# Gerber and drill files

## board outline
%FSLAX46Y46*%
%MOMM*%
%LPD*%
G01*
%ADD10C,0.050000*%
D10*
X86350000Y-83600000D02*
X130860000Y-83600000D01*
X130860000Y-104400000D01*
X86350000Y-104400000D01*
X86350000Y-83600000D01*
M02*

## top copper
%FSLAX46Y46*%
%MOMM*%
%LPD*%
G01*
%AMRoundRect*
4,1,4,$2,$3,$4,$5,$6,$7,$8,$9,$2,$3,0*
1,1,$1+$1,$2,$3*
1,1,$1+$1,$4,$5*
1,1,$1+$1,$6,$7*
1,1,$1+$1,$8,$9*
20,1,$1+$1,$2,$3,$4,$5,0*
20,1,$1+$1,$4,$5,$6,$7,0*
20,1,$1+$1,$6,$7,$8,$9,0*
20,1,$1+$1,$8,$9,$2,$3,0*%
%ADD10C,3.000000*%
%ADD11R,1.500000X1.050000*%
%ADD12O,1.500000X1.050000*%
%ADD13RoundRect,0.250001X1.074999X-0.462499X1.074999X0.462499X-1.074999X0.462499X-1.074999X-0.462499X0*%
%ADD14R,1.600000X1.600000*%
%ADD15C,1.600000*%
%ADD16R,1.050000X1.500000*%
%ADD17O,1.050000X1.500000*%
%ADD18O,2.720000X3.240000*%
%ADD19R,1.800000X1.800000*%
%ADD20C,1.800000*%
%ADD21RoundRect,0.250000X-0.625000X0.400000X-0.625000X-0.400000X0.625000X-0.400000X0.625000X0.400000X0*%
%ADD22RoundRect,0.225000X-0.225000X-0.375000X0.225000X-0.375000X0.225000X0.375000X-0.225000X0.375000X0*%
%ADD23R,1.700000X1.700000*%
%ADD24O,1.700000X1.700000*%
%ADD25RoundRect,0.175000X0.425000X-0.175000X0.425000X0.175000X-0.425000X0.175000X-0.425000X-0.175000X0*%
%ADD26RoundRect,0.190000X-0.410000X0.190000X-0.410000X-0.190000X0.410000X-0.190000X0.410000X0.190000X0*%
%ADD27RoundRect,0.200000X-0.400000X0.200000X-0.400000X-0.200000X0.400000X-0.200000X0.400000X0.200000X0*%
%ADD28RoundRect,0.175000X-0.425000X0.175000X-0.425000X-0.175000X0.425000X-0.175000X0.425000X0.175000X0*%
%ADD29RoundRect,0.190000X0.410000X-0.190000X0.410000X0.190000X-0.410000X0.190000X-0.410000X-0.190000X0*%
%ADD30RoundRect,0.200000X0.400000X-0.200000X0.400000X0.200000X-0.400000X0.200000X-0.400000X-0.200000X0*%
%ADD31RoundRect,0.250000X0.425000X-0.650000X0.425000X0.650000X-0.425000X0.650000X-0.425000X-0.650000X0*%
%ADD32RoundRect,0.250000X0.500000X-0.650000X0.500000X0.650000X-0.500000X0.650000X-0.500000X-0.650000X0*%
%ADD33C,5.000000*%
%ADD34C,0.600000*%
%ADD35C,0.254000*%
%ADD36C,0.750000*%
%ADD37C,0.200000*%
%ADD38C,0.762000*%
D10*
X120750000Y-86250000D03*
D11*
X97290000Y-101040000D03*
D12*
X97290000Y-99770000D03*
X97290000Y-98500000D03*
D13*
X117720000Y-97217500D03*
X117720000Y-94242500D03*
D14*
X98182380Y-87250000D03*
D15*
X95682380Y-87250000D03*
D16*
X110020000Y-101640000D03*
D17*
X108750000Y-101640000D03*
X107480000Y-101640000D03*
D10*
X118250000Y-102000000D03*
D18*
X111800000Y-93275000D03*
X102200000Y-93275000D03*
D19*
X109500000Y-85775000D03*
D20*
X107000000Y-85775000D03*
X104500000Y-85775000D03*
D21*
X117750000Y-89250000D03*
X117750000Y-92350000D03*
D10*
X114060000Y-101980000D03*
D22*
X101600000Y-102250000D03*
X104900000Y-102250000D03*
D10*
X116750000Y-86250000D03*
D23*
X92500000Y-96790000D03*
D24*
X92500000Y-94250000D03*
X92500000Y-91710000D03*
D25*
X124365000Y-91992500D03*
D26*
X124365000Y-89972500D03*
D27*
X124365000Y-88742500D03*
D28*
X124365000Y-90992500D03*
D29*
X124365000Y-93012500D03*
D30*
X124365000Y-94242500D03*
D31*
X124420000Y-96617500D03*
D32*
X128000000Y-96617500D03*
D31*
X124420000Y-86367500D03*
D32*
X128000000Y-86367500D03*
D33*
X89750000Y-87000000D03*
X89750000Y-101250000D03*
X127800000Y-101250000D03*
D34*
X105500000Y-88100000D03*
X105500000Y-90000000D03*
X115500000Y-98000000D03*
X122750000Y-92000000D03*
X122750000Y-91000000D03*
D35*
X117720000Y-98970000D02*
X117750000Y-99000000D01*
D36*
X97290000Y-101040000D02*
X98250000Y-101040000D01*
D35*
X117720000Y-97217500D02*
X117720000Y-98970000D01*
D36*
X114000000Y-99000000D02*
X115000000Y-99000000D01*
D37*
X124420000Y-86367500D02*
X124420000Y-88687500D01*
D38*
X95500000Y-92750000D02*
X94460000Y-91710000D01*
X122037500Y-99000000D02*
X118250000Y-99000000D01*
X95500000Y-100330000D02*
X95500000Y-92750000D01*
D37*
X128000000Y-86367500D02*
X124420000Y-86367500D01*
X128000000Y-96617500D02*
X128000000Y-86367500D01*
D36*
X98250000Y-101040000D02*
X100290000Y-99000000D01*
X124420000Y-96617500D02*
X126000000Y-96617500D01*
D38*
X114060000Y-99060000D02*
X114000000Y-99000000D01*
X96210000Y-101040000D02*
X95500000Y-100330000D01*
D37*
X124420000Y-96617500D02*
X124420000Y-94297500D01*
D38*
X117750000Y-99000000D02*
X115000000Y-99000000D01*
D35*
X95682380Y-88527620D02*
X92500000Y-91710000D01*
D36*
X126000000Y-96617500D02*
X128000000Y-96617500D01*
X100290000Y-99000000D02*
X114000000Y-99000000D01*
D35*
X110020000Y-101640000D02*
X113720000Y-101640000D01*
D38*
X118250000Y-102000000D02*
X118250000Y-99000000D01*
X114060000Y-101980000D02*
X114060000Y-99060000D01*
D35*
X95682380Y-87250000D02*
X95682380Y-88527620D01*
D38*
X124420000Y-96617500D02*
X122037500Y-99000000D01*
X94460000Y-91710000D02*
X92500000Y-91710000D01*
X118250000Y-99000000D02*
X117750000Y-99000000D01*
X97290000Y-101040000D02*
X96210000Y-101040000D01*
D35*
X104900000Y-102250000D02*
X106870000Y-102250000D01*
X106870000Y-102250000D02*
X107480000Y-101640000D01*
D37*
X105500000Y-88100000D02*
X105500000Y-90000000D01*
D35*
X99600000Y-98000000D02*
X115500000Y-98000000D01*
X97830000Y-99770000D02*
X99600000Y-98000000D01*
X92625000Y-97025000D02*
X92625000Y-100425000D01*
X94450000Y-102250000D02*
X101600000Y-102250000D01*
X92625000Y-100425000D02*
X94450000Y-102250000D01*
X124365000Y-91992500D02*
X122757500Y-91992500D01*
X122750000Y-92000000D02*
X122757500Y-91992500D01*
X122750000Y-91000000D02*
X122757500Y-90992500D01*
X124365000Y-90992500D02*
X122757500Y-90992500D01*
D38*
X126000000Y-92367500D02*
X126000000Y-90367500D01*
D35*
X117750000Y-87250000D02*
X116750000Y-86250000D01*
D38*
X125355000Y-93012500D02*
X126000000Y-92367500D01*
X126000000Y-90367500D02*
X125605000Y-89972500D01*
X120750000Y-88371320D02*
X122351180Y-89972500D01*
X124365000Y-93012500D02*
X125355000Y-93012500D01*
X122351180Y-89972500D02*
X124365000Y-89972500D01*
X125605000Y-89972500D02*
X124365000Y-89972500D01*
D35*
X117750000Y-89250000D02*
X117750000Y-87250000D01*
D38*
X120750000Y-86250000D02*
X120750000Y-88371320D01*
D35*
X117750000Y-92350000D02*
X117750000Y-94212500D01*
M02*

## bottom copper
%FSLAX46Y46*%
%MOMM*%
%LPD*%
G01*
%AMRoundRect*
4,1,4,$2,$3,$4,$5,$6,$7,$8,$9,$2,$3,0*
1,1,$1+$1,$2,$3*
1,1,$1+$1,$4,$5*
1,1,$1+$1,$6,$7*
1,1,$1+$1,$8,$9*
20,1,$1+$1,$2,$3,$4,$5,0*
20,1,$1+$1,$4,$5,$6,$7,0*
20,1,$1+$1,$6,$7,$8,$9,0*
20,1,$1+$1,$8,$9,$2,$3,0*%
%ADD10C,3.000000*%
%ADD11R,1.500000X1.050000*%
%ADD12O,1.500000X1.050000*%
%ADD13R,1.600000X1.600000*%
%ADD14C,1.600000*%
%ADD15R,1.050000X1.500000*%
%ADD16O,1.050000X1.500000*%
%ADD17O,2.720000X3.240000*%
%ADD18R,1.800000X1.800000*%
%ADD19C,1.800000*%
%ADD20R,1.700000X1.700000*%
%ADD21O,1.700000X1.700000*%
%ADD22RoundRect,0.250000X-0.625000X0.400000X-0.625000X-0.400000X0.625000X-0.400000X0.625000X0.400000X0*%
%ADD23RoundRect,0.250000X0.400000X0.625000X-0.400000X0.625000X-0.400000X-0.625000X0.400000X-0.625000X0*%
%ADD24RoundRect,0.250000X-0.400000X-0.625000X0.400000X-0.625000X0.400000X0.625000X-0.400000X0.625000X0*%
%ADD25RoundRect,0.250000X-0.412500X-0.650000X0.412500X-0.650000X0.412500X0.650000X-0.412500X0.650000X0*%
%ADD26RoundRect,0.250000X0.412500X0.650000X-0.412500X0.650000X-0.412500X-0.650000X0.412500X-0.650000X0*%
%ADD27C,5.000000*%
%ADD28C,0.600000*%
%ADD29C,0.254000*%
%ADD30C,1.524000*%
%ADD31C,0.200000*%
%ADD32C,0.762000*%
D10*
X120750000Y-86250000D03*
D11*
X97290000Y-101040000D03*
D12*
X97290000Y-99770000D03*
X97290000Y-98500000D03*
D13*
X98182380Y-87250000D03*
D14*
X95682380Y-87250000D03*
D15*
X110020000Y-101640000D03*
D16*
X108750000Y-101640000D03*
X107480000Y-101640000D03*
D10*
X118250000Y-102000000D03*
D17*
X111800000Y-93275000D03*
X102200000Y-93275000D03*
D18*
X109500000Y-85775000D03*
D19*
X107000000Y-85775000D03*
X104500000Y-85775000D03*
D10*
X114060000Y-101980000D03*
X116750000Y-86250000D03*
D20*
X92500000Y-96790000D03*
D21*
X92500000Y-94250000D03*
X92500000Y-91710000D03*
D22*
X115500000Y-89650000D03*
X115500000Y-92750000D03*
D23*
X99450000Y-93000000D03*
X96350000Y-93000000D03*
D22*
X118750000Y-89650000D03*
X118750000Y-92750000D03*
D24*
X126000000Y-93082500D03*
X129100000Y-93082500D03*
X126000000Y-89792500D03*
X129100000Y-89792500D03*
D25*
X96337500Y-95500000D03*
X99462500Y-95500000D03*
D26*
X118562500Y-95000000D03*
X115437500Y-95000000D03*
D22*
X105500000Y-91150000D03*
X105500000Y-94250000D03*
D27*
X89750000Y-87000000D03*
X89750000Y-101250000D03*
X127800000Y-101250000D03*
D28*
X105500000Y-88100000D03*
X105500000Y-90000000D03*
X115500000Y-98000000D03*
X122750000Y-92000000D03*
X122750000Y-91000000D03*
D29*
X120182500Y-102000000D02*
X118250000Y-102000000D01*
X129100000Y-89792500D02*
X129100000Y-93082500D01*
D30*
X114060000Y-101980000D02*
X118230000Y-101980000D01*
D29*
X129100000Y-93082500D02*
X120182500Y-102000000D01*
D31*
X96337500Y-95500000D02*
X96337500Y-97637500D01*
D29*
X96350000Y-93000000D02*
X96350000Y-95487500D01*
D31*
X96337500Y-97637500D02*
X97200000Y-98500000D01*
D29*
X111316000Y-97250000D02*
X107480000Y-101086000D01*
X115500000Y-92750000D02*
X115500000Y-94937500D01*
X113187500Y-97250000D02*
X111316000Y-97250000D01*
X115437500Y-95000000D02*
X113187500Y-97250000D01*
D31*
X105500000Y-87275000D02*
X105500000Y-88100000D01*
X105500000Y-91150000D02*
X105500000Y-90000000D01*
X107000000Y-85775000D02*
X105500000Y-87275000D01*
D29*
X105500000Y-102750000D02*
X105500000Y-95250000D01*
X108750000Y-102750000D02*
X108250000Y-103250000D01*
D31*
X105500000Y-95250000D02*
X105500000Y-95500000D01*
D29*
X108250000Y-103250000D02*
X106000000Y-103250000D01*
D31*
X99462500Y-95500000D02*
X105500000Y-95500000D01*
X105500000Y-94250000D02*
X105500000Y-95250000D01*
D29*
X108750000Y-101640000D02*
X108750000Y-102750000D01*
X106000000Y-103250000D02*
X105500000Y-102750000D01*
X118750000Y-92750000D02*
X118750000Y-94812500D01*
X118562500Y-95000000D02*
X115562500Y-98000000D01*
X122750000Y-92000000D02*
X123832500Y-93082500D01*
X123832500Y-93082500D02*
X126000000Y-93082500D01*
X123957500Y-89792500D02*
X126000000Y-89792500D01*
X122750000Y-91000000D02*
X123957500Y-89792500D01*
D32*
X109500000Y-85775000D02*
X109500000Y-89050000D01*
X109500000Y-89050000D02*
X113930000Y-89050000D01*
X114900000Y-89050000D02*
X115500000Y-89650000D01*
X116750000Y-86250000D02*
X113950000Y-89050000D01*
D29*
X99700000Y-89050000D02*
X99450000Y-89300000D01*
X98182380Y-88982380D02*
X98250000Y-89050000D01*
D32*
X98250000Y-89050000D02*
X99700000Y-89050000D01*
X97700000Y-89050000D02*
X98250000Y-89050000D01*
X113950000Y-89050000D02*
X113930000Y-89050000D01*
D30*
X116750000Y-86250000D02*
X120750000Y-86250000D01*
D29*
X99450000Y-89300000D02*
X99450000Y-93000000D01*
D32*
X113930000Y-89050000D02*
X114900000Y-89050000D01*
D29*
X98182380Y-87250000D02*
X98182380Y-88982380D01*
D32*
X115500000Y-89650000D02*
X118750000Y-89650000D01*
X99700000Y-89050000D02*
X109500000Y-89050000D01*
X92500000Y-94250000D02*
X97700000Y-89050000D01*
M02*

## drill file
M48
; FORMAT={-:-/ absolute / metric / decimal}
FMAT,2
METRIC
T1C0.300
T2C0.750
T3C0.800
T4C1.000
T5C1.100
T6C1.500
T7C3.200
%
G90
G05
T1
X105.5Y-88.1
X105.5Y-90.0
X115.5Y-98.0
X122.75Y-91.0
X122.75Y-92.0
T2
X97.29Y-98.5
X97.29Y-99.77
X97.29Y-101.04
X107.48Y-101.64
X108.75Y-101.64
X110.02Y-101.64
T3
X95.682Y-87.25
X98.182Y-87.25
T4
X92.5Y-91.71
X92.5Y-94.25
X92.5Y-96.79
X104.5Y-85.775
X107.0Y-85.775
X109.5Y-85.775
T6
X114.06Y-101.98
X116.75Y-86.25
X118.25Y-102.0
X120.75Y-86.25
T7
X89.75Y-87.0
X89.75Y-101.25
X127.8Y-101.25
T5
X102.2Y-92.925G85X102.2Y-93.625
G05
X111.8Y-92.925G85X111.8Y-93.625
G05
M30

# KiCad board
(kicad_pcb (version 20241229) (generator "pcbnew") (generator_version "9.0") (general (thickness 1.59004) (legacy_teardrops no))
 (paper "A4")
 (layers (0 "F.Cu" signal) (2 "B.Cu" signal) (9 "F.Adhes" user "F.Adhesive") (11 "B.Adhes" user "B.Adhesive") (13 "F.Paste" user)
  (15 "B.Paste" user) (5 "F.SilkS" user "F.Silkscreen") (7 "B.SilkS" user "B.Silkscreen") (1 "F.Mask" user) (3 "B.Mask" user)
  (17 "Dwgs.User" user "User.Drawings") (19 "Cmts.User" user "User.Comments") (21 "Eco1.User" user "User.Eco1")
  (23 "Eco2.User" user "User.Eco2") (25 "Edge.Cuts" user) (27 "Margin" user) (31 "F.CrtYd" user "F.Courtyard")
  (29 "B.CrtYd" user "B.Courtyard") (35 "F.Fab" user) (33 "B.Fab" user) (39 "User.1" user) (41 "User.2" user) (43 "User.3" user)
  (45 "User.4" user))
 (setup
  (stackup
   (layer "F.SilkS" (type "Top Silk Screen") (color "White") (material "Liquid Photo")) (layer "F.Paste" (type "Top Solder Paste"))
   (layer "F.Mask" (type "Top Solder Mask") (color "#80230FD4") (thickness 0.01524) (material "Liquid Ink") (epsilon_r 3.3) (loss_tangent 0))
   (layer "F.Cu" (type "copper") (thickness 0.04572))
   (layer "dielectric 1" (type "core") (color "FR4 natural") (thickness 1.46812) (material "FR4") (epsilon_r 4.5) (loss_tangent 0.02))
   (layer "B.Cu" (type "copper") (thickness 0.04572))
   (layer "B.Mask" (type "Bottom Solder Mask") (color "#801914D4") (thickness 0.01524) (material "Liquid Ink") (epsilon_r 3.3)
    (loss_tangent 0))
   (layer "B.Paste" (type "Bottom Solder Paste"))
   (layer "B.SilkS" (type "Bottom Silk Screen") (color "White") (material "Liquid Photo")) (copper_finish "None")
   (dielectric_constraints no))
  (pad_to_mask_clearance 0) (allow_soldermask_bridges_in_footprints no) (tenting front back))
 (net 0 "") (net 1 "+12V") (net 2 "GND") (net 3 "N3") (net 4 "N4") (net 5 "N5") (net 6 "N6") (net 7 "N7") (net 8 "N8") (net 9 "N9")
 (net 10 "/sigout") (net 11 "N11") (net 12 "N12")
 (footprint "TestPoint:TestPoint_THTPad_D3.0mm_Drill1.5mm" (layer "F.Cu") (at 120.75 86.25)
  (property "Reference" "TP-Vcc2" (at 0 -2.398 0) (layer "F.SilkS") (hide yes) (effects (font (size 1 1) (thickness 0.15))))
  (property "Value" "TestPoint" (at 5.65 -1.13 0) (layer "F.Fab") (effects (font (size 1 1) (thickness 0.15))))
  (pad "1" thru_hole circle (at 0 0) (size 3 3) (drill 1.5) (layers "*.Cu" "*.Mask") (remove_unused_layers no) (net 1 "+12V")))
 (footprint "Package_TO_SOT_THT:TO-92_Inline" (layer "F.Cu") (at 97.29 101.04 90)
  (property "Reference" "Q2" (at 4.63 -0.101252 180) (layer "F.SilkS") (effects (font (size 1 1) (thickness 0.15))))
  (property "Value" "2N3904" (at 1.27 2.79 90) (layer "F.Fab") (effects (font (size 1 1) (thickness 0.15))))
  (pad "1" thru_hole rect (at 0 0 90) (size 1.05 1.5) (drill 0.75) (layers "*.Cu" "*.Mask") (remove_unused_layers no) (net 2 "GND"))
  (pad "2" thru_hole oval (at 1.27 0 90) (size 1.05 1.5) (drill 0.75) (layers "*.Cu" "*.Mask") (remove_unused_layers no) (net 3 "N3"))
  (pad "3" thru_hole oval (at 2.54 0 90) (size 1.05 1.5) (drill 0.75) (layers "*.Cu" "*.Mask") (remove_unused_layers no) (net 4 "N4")))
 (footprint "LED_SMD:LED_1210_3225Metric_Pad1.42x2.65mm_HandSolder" (layer "F.Cu") (at 117.72 95.73 90)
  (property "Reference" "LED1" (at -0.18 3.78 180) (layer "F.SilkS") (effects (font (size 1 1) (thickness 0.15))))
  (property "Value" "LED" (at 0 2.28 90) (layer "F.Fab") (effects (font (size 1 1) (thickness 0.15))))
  (pad "1" smd roundrect (at -1.4875 0 90) (size 1.425 2.65) (layers "F.Cu" "F.Mask" "F.Paste") (roundrect_rratio 0.175439) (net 2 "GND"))
  (pad "2" smd roundrect (at 1.4875 0 90) (size 1.425 2.65) (layers "F.Cu" "F.Mask" "F.Paste") (roundrect_rratio 0.175439) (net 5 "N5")))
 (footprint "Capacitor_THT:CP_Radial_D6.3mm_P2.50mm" (layer "F.Cu") (at 98.18238 87.25 180)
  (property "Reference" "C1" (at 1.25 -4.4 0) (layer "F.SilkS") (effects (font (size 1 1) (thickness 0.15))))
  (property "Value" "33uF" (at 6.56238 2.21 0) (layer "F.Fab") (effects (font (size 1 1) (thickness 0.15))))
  (pad "1" thru_hole rect (at 0 0 180) (size 1.6 1.6) (drill 0.8) (layers "*.Cu" "*.Mask") (remove_unused_layers no) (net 1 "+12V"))
  (pad "2" thru_hole circle (at 2.5 0 180) (size 1.6 1.6) (drill 0.8) (layers "*.Cu" "*.Mask") (remove_unused_layers no) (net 2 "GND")))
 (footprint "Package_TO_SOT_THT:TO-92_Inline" (layer "F.Cu") (at 110.02 101.64 180)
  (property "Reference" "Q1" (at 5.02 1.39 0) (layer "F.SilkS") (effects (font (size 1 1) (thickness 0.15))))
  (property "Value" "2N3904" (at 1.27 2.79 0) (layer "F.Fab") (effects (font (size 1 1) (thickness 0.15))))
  (pad "1" thru_hole rect (at 0 0 180) (size 1.05 1.5) (drill 0.75) (layers "*.Cu" "*.Mask") (remove_unused_layers no) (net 2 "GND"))
  (pad "2" thru_hole oval (at 1.27 0 180) (size 1.05 1.5) (drill 0.75) (layers "*.Cu" "*.Mask") (remove_unused_layers no) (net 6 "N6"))
  (pad "3" thru_hole oval (at 2.54 0 180) (size 1.05 1.5) (drill 0.75) (layers "*.Cu" "*.Mask") (remove_unused_layers no) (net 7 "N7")))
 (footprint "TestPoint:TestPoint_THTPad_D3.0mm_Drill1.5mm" (layer "F.Cu") (at 118.25 102)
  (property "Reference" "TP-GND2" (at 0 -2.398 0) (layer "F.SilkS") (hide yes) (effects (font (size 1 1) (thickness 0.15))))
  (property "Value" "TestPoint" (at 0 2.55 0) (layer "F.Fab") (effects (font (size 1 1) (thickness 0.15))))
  (pad "1" thru_hole circle (at 0 0) (size 3 3) (drill 1.5) (layers "*.Cu" "*.Mask") (remove_unused_layers no) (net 2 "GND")))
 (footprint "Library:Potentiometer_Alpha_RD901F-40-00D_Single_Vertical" (layer "F.Cu") (at 109.5 85.775 -90)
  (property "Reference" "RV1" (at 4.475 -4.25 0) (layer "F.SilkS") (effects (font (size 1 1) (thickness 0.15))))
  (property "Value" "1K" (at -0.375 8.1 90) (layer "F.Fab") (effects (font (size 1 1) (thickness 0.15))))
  (pad "" thru_hole oval (at 7.5 -2.3) (size 2.72 3.24) (drill oval 1.1 1.8) (layers "*.Cu" "*.Mask") (remove_unused_layers no))
  (pad "" thru_hole oval (at 7.5 7.3) (size 2.72 3.24) (drill oval 1.1 1.8) (layers "*.Cu" "*.Mask") (remove_unused_layers no))
  (pad "1" thru_hole rect (at 0 0) (size 1.8 1.8) (drill 1) (layers "*.Cu" "*.Mask") (remove_unused_layers no) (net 1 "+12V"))
  (pad "2" thru_hole circle (at 0 2.5) (size 1.8 1.8) (drill 1) (layers "*.Cu" "*.Mask") (remove_unused_layers no) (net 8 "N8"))
  (pad "3" thru_hole circle (at 0 5) (size 1.8 1.8) (drill 1) (layers "*.Cu" "*.Mask") (remove_unused_layers no) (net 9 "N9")))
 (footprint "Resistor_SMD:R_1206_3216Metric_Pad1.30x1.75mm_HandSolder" (layer "F.Cu") (at 117.75 90.8 -90)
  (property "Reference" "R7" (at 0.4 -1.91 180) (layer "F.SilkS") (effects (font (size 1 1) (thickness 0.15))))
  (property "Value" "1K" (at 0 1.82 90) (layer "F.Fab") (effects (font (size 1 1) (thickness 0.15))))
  (pad "1" smd roundrect (at -1.55 0 270) (size 1.3 1.75) (layers "F.Cu" "F.Mask" "F.Paste") (roundrect_rratio 0.192308) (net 1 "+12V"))
  (pad "2" smd roundrect (at 1.55 0 270) (size 1.3 1.75) (layers "F.Cu" "F.Mask" "F.Paste") (roundrect_rratio 0.192308) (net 5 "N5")))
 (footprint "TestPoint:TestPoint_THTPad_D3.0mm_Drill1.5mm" (layer "F.Cu") (at 114.06 101.98)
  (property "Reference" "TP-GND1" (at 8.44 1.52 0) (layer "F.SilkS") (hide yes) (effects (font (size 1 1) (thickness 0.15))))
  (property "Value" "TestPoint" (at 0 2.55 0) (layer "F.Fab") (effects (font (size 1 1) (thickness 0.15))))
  (pad "1" thru_hole circle (at 0 0) (size 3 3) (drill 1.5) (layers "*.Cu" "*.Mask") (remove_unused_layers no) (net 2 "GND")))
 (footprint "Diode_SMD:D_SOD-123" (layer "F.Cu") (at 103.25 102.25)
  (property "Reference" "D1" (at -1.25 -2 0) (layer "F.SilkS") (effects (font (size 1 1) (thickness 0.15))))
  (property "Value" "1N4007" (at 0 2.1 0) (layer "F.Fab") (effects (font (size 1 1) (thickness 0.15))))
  (pad "1" smd roundrect (at -1.65 0) (size 0.9 1.2) (layers "F.Cu" "F.Mask" "F.Paste") (roundrect_rratio 0.25) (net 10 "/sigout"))
  (pad "2" smd roundrect (at 1.65 0) (size 0.9 1.2) (layers "F.Cu" "F.Mask" "F.Paste") (roundrect_rratio 0.25) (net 7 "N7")))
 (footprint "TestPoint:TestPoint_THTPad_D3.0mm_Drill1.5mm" (layer "F.Cu") (at 116.75 86.25)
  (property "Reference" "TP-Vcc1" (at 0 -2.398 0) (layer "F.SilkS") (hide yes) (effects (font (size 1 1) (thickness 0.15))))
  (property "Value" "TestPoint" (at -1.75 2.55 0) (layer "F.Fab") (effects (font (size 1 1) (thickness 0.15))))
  (pad "1" thru_hole circle (at 0 0) (size 3 3) (drill 1.5) (layers "*.Cu" "*.Mask") (remove_unused_layers no) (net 1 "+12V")))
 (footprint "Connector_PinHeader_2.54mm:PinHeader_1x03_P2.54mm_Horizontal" (layer "F.Cu") (at 92.5 96.79 180)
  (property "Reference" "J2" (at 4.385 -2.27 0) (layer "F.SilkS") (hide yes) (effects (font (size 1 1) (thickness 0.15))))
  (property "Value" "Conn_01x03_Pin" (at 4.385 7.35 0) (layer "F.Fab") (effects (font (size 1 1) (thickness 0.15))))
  (pad "1" thru_hole rect (at 0 0 180) (size 1.7 1.7) (drill 1) (layers "*.Cu" "*.Mask") (remove_unused_layers no) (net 10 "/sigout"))
  (pad "2" thru_hole oval (at 0 2.54 180) (size 1.7 1.7) (drill 1) (layers "*.Cu" "*.Mask") (remove_unused_layers no) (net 1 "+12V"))
  (pad "3" thru_hole oval (at 0 5.08 180) (size 1.7 1.7) (drill 1) (layers "*.Cu" "*.Mask") (remove_unused_layers no) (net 2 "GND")))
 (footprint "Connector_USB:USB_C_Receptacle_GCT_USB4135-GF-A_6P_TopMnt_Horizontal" (layer "F.Cu") (at 127.3975 91.4925 90)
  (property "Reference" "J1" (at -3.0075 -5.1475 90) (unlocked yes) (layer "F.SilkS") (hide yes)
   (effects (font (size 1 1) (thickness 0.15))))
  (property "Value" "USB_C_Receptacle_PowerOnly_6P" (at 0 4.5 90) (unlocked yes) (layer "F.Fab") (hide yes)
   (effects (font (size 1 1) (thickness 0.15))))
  (pad "A5" smd roundrect (at -0.5 -3.0325 90) (size 0.7 1.2) (layers "F.Cu" "F.Mask" "F.Paste") (roundrect_rratio 0.25) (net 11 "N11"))
  (pad "A9" smd roundrect (at 1.52 -3.0325 270) (size 0.76 1.2) (layers "F.Cu" "F.Mask" "F.Paste") (roundrect_rratio 0.25) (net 1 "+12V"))
  (pad "A12" smd roundrect (at 2.75 -3.0325 270) (size 0.8 1.2) (layers "F.Cu" "F.Mask" "F.Paste") (roundrect_rratio 0.25) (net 2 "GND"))
  (pad "B5" smd roundrect (at 0.5 -3.0325 270) (size 0.7 1.2) (layers "F.Cu" "F.Mask" "F.Paste") (roundrect_rratio 0.25) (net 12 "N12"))
  (pad "B9" smd roundrect (at -1.52 -3.0325 90) (size 0.76 1.2) (layers "F.Cu" "F.Mask" "F.Paste") (roundrect_rratio 0.25) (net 1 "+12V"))
  (pad "B12" smd roundrect (at -2.75 -3.0325 90) (size 0.8 1.2) (layers "F.Cu" "F.Mask" "F.Paste") (roundrect_rratio 0.25) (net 2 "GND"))
  (pad "S1" smd roundrect (at -5.125 -2.9775 90) (size 1.8 1.35) (layers "F.Cu" "F.Mask" "F.Paste") (roundrect_rratio 0.1851851852)
   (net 2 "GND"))
  (pad "S1" smd roundrect (at -5.125 0.6025 90) (size 1.8 1.5) (layers "F.Cu" "F.Mask" "F.Paste") (roundrect_rratio 0.1666666667)
   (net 2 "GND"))
  (pad "S1" smd roundrect (at 5.125 -2.9775 90) (size 1.8 1.35) (layers "F.Cu" "F.Mask" "F.Paste") (roundrect_rratio 0.1851851852)
   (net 2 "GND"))
  (pad "S1" smd roundrect (at 5.125 0.6025 90) (size 1.8 1.5) (layers "F.Cu" "F.Mask" "F.Paste") (roundrect_rratio 0.1666666667)
   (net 2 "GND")))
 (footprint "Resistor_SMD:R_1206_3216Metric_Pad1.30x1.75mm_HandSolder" (layer "B.Cu") (at 115.5 91.2 -90)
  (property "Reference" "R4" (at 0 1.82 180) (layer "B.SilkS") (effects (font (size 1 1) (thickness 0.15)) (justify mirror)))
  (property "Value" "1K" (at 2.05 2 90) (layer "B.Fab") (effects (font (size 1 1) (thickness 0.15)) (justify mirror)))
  (pad "1" smd roundrect (at -1.55 0 270) (size 1.3 1.75) (layers "B.Cu" "B.Mask" "B.Paste") (roundrect_rratio 0.192308) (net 1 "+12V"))
  (pad "2" smd roundrect (at 1.55 0 270) (size 1.3 1.75) (layers "B.Cu" "B.Mask" "B.Paste") (roundrect_rratio 0.192308) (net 7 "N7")))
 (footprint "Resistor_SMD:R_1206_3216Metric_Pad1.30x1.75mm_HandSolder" (layer "B.Cu") (at 97.9 93 180)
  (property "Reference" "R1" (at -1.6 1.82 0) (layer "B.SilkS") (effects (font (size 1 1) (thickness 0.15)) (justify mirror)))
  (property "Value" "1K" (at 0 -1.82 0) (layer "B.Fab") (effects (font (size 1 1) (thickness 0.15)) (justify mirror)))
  (pad "1" smd roundrect (at -1.55 0 180) (size 1.3 1.75) (layers "B.Cu" "B.Mask" "B.Paste") (roundrect_rratio 0.192308) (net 1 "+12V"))
  (pad "2" smd roundrect (at 1.55 0 180) (size 1.3 1.75) (layers "B.Cu" "B.Mask" "B.Paste") (roundrect_rratio 0.192308) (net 4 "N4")))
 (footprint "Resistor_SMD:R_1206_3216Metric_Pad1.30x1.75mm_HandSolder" (layer "B.Cu") (at 118.75 91.2 -90)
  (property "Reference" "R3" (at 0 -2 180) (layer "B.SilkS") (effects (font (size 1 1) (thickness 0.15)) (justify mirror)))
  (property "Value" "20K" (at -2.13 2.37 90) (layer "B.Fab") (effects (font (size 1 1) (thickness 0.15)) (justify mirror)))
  (pad "1" smd roundrect (at -1.55 0 270) (size 1.3 1.75) (layers "B.Cu" "B.Mask" "B.Paste") (roundrect_rratio 0.192308) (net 1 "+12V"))
  (pad "2" smd roundrect (at 1.55 0 270) (size 1.3 1.75) (layers "B.Cu" "B.Mask" "B.Paste") (roundrect_rratio 0.192308) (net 3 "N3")))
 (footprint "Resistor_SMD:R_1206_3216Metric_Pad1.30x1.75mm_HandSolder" (layer "B.Cu") (at 127.55 93.0825)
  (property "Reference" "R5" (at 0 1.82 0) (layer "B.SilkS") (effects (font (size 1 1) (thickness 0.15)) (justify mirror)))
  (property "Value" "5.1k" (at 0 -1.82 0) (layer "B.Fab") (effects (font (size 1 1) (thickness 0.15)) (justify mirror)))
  (pad "1" smd roundrect (at -1.55 0) (size 1.3 1.75) (layers "B.Cu" "B.Mask" "B.Paste") (roundrect_rratio 0.192308) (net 11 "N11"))
  (pad "2" smd roundrect (at 1.55 0) (size 1.3 1.75) (layers "B.Cu" "B.Mask" "B.Paste") (roundrect_rratio 0.192308) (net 2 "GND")))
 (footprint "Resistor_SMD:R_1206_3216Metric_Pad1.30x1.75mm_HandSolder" (layer "B.Cu") (at 127.55 89.7925)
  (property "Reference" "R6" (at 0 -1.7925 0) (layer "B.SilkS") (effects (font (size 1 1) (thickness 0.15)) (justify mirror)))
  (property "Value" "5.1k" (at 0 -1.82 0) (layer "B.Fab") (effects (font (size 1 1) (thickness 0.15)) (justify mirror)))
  (pad "1" smd roundrect (at -1.55 0) (size 1.3 1.75) (layers "B.Cu" "B.Mask" "B.Paste") (roundrect_rratio 0.192308) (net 12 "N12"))
  (pad "2" smd roundrect (at 1.55 0) (size 1.3 1.75) (layers "B.Cu" "B.Mask" "B.Paste") (roundrect_rratio 0.192308) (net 2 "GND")))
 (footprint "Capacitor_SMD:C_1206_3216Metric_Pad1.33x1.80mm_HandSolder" (layer "B.Cu") (at 97.9 95.5)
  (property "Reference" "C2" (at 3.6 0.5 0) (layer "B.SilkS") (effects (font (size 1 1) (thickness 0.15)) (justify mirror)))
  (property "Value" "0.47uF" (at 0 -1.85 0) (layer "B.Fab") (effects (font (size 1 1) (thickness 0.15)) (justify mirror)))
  (pad "1" smd roundrect (at -1.5625 0) (size 1.325 1.8) (layers "B.Cu" "B.Mask" "B.Paste") (roundrect_rratio 0.188679) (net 4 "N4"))
  (pad "2" smd roundrect (at 1.5625 0) (size 1.325 1.8) (layers "B.Cu" "B.Mask" "B.Paste") (roundrect_rratio 0.188679) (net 6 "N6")))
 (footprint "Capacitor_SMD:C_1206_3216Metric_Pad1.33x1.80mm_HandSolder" (layer "B.Cu") (at 117 95 180)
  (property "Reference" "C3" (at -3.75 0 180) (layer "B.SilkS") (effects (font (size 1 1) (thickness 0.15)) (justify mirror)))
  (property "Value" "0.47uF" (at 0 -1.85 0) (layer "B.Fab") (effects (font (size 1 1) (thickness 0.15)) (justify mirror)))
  (pad "1" smd roundrect (at -1.5625 0 180) (size 1.325 1.8) (layers "B.Cu" "B.Mask" "B.Paste") (roundrect_rratio 0.188679) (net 3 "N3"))
  (pad "2" smd roundrect (at 1.5625 0 180) (size 1.325 1.8) (layers "B.Cu" "B.Mask" "B.Paste") (roundrect_rratio 0.188679) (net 7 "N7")))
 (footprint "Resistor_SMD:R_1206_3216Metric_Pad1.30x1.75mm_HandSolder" (layer "B.Cu") (at 105.5 92.7 -90)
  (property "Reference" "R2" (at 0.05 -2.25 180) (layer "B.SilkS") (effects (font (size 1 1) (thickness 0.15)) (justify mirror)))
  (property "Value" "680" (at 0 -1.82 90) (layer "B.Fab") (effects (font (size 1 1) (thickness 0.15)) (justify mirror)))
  (pad "1" smd roundrect (at -1.55 0 270) (size 1.3 1.75) (layers "B.Cu" "B.Mask" "B.Paste") (roundrect_rratio 0.192308) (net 8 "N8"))
  (pad "2" smd roundrect (at 1.55 0 270) (size 1.3 1.75) (layers "B.Cu" "B.Mask" "B.Paste") (roundrect_rratio 0.192308) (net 6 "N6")))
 (gr_rect (start 86.35 83.6) (end 130.86 104.4) (stroke (width 0.05) (type default)) (fill no) (layer "Edge.Cuts"))
 (via (at 89.75 87) (size 5) (drill 3.2) (layers "F.Cu" "B.Cu") (free yes) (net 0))
 (via (at 89.75 101.25) (size 5) (drill 3.2) (layers "F.Cu" "B.Cu") (free yes) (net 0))
 (via (at 127.8 101.25) (size 5) (drill 3.2) (layers "F.Cu" "B.Cu") (free yes) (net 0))
 (segment (start 117.72 98.97) (end 117.75 99) (width 0.254) (layer "F.Cu") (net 2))
 (segment (start 97.29 101.04) (end 98.25 101.04) (width 0.75) (layer "F.Cu") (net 2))
 (segment (start 117.72 97.2175) (end 117.72 98.97) (width 0.254) (layer "F.Cu") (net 2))
 (segment (start 114 99) (end 115 99) (width 0.75) (layer "F.Cu") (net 2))
 (segment (start 124.42 86.3675) (end 124.42 88.6875) (width 0.2) (layer "F.Cu") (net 2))
 (segment (start 95.5 92.75) (end 94.46 91.71) (width 0.762) (layer "F.Cu") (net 2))
 (segment (start 122.0375 99) (end 118.25 99) (width 0.762) (layer "F.Cu") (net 2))
 (segment (start 95.5 100.33) (end 95.5 92.75) (width 0.762) (layer "F.Cu") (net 2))
 (segment (start 128 86.3675) (end 124.42 86.3675) (width 0.2) (layer "F.Cu") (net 2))
 (segment (start 128 96.6175) (end 128 86.3675) (width 0.2) (layer "F.Cu") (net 2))
 (segment (start 98.25 101.04) (end 100.29 99) (width 0.75) (layer "F.Cu") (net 2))
 (segment (start 124.42 96.6175) (end 126 96.6175) (width 0.75) (layer "F.Cu") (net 2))
 (segment (start 114.06 99.06) (end 114 99) (width 0.762) (layer "F.Cu") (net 2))
 (segment (start 96.21 101.04) (end 95.5 100.33) (width 0.762) (layer "F.Cu") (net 2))
 (segment (start 124.42 96.6175) (end 124.42 94.2975) (width 0.2) (layer "F.Cu") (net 2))
 (segment (start 117.75 99) (end 115 99) (width 0.762) (layer "F.Cu") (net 2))
 (segment (start 95.68238 88.52762) (end 92.5 91.71) (width 0.254) (layer "F.Cu") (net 2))
 (segment (start 126 96.6175) (end 128 96.6175) (width 0.75) (layer "F.Cu") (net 2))
 (segment (start 100.29 99) (end 114 99) (width 0.75) (layer "F.Cu") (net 2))
 (segment (start 110.02 101.64) (end 113.72 101.64) (width 0.254) (layer "F.Cu") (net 2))
 (segment (start 118.25 102) (end 118.25 99) (width 0.762) (layer "F.Cu") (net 2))
 (segment (start 114.06 101.98) (end 114.06 99.06) (width 0.762) (layer "F.Cu") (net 2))
 (segment (start 95.68238 87.25) (end 95.68238 88.52762) (width 0.254) (layer "F.Cu") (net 2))
 (segment (start 124.42 96.6175) (end 122.0375 99) (width 0.762) (layer "F.Cu") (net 2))
 (segment (start 94.46 91.71) (end 92.5 91.71) (width 0.762) (layer "F.Cu") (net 2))
 (segment (start 118.25 99) (end 117.75 99) (width 0.762) (layer "F.Cu") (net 2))
 (segment (start 97.29 101.04) (end 96.21 101.04) (width 0.762) (layer "F.Cu") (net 2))
 (segment (start 120.1825 102) (end 118.25 102) (width 0.254) (layer "B.Cu") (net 2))
 (segment (start 129.1 89.7925) (end 129.1 93.0825) (width 0.254) (layer "B.Cu") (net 2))
 (segment (start 114.06 101.98) (end 118.23 101.98) (width 1.524) (layer "B.Cu") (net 2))
 (segment (start 129.1 93.0825) (end 120.1825 102) (width 0.254) (layer "B.Cu") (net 2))
 (segment (start 96.3375 95.5) (end 96.3375 97.6375) (width 0.2) (layer "B.Cu") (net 4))
 (segment (start 96.35 93) (end 96.35 95.4875) (width 0.254) (layer "B.Cu") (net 4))
 (segment (start 96.3375 97.6375) (end 97.2 98.5) (width 0.2) (layer "B.Cu") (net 4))
 (segment (start 104.9 102.25) (end 106.87 102.25) (width 0.254) (layer "F.Cu") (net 7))
 (segment (start 106.87 102.25) (end 107.48 101.64) (width 0.254) (layer "F.Cu") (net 7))
 (segment (start 111.316 97.25) (end 107.48 101.086) (width 0.254) (layer "B.Cu") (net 7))
 (segment (start 115.5 92.75) (end 115.5 94.9375) (width 0.254) (layer "B.Cu") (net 7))
 (segment (start 113.1875 97.25) (end 111.316 97.25) (width 0.254) (layer "B.Cu") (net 7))
 (segment (start 115.4375 95) (end 113.1875 97.25) (width 0.254) (layer "B.Cu") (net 7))
 (segment (start 105.5 88.1) (end 105.5 90) (width 0.2) (layer "F.Cu") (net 8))
 (via (at 105.5 88.1) (size 0.6) (drill 0.3) (layers "F.Cu" "B.Cu") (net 8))
 (via (at 105.5 90) (size 0.6) (drill 0.3) (layers "F.Cu" "B.Cu") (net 8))
 (segment (start 105.5 87.275) (end 105.5 88.1) (width 0.2) (layer "B.Cu") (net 8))
 (segment (start 105.5 91.15) (end 105.5 90) (width 0.2) (layer "B.Cu") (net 8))
 (segment (start 107 85.775) (end 105.5 87.275) (width 0.2) (layer "B.Cu") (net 8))
 (segment (start 105.5 102.75) (end 105.5 95.25) (width 0.254) (layer "B.Cu") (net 6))
 (segment (start 108.75 102.75) (end 108.25 103.25) (width 0.254) (layer "B.Cu") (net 6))
 (segment (start 105.5 95.25) (end 105.5 95.5) (width 0.2) (layer "B.Cu") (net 6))
 (segment (start 108.25 103.25) (end 106 103.25) (width 0.254) (layer "B.Cu") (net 6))
 (segment (start 99.4625 95.5) (end 105.5 95.5) (width 0.2) (layer "B.Cu") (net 6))
 (segment (start 105.5 94.25) (end 105.5 95.25) (width 0.2) (layer "B.Cu") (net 6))
 (segment (start 108.75 101.64) (end 108.75 102.75) (width 0.254) (layer "B.Cu") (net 6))
 (segment (start 106 103.25) (end 105.5 102.75) (width 0.254) (layer "B.Cu") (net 6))
 (segment (start 99.6 98) (end 115.5 98) (width 0.254) (layer "F.Cu") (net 3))
 (segment (start 97.83 99.77) (end 99.6 98) (width 0.254) (layer "F.Cu") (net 3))
 (via (at 115.5 98) (size 0.6) (drill 0.3) (layers "F.Cu" "B.Cu") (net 3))
 (segment (start 118.75 92.75) (end 118.75 94.8125) (width 0.254) (layer "B.Cu") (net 3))
 (segment (start 118.5625 95) (end 115.5625 98) (width 0.254) (layer "B.Cu") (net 3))
 (segment (start 92.625 97.025) (end 92.625 100.425) (width 0.254) (layer "F.Cu") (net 10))
 (segment (start 94.45 102.25) (end 101.6 102.25) (width 0.254) (layer "F.Cu") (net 10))
 (segment (start 92.625 100.425) (end 94.45 102.25) (width 0.254) (layer "F.Cu") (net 10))
 (segment (start 124.365 91.9925) (end 122.7575 91.9925) (width 0.254) (layer "F.Cu") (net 11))
 (segment (start 122.75 92) (end 122.7575 91.9925) (width 0.254) (layer "F.Cu") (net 11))
 (via (at 122.75 92) (size 0.6) (drill 0.3) (layers "F.Cu" "B.Cu") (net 11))
 (segment (start 122.75 92) (end 123.8325 93.0825) (width 0.254) (layer "B.Cu") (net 11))
 (segment (start 123.8325 93.0825) (end 126 93.0825) (width 0.254) (layer "B.Cu") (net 11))
 (segment (start 122.75 91) (end 122.7575 90.9925) (width 0.254) (layer "F.Cu") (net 12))
 (segment (start 124.365 90.9925) (end 122.7575 90.9925) (width 0.254) (layer "F.Cu") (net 12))
 (via (at 122.75 91) (size 0.6) (drill 0.3) (layers "F.Cu" "B.Cu") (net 12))
 (segment (start 123.9575 89.7925) (end 126 89.7925) (width 0.254) (layer "B.Cu") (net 12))
 (segment (start 122.75 91) (end 123.9575 89.7925) (width 0.254) (layer "B.Cu") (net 12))
 (segment (start 126 92.3675) (end 126 90.3675) (width 0.762) (layer "F.Cu") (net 1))
 (segment (start 117.75 87.25) (end 116.75 86.25) (width 0.254) (layer "F.Cu") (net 1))
 (segment (start 125.355 93.0125) (end 126 92.3675) (width 0.762) (layer "F.Cu") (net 1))
 (segment (start 126 90.3675) (end 125.605 89.9725) (width 0.762) (layer "F.Cu") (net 1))
 (segment (start 120.75 88.37132) (end 122.35118 89.9725) (width 0.762) (layer "F.Cu") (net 1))
 (segment (start 124.365 93.0125) (end 125.355 93.0125) (width 0.762) (layer "F.Cu") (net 1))
 (segment (start 122.35118 89.9725) (end 124.365 89.9725) (width 0.762) (layer "F.Cu") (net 1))
 (segment (start 125.605 89.9725) (end 124.365 89.9725) (width 0.762) (layer "F.Cu") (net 1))
 (segment (start 117.75 89.25) (end 117.75 87.25) (width 0.254) (layer "F.Cu") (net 1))
 (segment (start 120.75 86.25) (end 120.75 88.37132) (width 0.762) (layer "F.Cu") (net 1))
 (segment (start 109.5 85.775) (end 109.5 89.05) (width 0.762) (layer "B.Cu") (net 1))
 (segment (start 109.5 89.05) (end 113.93 89.05) (width 0.762) (layer "B.Cu") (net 1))
 (segment (start 114.9 89.05) (end 115.5 89.65) (width 0.762) (layer "B.Cu") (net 1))
 (segment (start 116.75 86.25) (end 113.95 89.05) (width 0.762) (layer "B.Cu") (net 1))
 (segment (start 99.7 89.05) (end 99.45 89.3) (width 0.254) (layer "B.Cu") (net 1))
 (segment (start 98.18238 88.98238) (end 98.25 89.05) (width 0.254) (layer "B.Cu") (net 1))
 (segment (start 98.25 89.05) (end 99.7 89.05) (width 0.762) (layer "B.Cu") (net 1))
 (segment (start 97.7 89.05) (end 98.25 89.05) (width 0.762) (layer "B.Cu") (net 1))
 (segment (start 113.95 89.05) (end 113.93 89.05) (width 0.762) (layer "B.Cu") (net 1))
 (segment (start 116.75 86.25) (end 120.75 86.25) (width 1.524) (layer "B.Cu") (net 1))
 (segment (start 99.45 89.3) (end 99.45 93) (width 0.254) (layer "B.Cu") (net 1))
 (segment (start 113.93 89.05) (end 114.9 89.05) (width 0.762) (layer "B.Cu") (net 1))
 (segment (start 98.18238 87.25) (end 98.18238 88.98238) (width 0.254) (layer "B.Cu") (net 1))
 (segment (start 115.5 89.65) (end 118.75 89.65) (width 0.762) (layer "B.Cu") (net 1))
 (segment (start 99.7 89.05) (end 109.5 89.05) (width 0.762) (layer "B.Cu") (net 1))
 (segment (start 92.5 94.25) (end 97.7 89.05) (width 0.762) (layer "B.Cu") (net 1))
 (segment (start 117.75 92.35) (end 117.75 94.2125) (width 0.254) (layer "F.Cu") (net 5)))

